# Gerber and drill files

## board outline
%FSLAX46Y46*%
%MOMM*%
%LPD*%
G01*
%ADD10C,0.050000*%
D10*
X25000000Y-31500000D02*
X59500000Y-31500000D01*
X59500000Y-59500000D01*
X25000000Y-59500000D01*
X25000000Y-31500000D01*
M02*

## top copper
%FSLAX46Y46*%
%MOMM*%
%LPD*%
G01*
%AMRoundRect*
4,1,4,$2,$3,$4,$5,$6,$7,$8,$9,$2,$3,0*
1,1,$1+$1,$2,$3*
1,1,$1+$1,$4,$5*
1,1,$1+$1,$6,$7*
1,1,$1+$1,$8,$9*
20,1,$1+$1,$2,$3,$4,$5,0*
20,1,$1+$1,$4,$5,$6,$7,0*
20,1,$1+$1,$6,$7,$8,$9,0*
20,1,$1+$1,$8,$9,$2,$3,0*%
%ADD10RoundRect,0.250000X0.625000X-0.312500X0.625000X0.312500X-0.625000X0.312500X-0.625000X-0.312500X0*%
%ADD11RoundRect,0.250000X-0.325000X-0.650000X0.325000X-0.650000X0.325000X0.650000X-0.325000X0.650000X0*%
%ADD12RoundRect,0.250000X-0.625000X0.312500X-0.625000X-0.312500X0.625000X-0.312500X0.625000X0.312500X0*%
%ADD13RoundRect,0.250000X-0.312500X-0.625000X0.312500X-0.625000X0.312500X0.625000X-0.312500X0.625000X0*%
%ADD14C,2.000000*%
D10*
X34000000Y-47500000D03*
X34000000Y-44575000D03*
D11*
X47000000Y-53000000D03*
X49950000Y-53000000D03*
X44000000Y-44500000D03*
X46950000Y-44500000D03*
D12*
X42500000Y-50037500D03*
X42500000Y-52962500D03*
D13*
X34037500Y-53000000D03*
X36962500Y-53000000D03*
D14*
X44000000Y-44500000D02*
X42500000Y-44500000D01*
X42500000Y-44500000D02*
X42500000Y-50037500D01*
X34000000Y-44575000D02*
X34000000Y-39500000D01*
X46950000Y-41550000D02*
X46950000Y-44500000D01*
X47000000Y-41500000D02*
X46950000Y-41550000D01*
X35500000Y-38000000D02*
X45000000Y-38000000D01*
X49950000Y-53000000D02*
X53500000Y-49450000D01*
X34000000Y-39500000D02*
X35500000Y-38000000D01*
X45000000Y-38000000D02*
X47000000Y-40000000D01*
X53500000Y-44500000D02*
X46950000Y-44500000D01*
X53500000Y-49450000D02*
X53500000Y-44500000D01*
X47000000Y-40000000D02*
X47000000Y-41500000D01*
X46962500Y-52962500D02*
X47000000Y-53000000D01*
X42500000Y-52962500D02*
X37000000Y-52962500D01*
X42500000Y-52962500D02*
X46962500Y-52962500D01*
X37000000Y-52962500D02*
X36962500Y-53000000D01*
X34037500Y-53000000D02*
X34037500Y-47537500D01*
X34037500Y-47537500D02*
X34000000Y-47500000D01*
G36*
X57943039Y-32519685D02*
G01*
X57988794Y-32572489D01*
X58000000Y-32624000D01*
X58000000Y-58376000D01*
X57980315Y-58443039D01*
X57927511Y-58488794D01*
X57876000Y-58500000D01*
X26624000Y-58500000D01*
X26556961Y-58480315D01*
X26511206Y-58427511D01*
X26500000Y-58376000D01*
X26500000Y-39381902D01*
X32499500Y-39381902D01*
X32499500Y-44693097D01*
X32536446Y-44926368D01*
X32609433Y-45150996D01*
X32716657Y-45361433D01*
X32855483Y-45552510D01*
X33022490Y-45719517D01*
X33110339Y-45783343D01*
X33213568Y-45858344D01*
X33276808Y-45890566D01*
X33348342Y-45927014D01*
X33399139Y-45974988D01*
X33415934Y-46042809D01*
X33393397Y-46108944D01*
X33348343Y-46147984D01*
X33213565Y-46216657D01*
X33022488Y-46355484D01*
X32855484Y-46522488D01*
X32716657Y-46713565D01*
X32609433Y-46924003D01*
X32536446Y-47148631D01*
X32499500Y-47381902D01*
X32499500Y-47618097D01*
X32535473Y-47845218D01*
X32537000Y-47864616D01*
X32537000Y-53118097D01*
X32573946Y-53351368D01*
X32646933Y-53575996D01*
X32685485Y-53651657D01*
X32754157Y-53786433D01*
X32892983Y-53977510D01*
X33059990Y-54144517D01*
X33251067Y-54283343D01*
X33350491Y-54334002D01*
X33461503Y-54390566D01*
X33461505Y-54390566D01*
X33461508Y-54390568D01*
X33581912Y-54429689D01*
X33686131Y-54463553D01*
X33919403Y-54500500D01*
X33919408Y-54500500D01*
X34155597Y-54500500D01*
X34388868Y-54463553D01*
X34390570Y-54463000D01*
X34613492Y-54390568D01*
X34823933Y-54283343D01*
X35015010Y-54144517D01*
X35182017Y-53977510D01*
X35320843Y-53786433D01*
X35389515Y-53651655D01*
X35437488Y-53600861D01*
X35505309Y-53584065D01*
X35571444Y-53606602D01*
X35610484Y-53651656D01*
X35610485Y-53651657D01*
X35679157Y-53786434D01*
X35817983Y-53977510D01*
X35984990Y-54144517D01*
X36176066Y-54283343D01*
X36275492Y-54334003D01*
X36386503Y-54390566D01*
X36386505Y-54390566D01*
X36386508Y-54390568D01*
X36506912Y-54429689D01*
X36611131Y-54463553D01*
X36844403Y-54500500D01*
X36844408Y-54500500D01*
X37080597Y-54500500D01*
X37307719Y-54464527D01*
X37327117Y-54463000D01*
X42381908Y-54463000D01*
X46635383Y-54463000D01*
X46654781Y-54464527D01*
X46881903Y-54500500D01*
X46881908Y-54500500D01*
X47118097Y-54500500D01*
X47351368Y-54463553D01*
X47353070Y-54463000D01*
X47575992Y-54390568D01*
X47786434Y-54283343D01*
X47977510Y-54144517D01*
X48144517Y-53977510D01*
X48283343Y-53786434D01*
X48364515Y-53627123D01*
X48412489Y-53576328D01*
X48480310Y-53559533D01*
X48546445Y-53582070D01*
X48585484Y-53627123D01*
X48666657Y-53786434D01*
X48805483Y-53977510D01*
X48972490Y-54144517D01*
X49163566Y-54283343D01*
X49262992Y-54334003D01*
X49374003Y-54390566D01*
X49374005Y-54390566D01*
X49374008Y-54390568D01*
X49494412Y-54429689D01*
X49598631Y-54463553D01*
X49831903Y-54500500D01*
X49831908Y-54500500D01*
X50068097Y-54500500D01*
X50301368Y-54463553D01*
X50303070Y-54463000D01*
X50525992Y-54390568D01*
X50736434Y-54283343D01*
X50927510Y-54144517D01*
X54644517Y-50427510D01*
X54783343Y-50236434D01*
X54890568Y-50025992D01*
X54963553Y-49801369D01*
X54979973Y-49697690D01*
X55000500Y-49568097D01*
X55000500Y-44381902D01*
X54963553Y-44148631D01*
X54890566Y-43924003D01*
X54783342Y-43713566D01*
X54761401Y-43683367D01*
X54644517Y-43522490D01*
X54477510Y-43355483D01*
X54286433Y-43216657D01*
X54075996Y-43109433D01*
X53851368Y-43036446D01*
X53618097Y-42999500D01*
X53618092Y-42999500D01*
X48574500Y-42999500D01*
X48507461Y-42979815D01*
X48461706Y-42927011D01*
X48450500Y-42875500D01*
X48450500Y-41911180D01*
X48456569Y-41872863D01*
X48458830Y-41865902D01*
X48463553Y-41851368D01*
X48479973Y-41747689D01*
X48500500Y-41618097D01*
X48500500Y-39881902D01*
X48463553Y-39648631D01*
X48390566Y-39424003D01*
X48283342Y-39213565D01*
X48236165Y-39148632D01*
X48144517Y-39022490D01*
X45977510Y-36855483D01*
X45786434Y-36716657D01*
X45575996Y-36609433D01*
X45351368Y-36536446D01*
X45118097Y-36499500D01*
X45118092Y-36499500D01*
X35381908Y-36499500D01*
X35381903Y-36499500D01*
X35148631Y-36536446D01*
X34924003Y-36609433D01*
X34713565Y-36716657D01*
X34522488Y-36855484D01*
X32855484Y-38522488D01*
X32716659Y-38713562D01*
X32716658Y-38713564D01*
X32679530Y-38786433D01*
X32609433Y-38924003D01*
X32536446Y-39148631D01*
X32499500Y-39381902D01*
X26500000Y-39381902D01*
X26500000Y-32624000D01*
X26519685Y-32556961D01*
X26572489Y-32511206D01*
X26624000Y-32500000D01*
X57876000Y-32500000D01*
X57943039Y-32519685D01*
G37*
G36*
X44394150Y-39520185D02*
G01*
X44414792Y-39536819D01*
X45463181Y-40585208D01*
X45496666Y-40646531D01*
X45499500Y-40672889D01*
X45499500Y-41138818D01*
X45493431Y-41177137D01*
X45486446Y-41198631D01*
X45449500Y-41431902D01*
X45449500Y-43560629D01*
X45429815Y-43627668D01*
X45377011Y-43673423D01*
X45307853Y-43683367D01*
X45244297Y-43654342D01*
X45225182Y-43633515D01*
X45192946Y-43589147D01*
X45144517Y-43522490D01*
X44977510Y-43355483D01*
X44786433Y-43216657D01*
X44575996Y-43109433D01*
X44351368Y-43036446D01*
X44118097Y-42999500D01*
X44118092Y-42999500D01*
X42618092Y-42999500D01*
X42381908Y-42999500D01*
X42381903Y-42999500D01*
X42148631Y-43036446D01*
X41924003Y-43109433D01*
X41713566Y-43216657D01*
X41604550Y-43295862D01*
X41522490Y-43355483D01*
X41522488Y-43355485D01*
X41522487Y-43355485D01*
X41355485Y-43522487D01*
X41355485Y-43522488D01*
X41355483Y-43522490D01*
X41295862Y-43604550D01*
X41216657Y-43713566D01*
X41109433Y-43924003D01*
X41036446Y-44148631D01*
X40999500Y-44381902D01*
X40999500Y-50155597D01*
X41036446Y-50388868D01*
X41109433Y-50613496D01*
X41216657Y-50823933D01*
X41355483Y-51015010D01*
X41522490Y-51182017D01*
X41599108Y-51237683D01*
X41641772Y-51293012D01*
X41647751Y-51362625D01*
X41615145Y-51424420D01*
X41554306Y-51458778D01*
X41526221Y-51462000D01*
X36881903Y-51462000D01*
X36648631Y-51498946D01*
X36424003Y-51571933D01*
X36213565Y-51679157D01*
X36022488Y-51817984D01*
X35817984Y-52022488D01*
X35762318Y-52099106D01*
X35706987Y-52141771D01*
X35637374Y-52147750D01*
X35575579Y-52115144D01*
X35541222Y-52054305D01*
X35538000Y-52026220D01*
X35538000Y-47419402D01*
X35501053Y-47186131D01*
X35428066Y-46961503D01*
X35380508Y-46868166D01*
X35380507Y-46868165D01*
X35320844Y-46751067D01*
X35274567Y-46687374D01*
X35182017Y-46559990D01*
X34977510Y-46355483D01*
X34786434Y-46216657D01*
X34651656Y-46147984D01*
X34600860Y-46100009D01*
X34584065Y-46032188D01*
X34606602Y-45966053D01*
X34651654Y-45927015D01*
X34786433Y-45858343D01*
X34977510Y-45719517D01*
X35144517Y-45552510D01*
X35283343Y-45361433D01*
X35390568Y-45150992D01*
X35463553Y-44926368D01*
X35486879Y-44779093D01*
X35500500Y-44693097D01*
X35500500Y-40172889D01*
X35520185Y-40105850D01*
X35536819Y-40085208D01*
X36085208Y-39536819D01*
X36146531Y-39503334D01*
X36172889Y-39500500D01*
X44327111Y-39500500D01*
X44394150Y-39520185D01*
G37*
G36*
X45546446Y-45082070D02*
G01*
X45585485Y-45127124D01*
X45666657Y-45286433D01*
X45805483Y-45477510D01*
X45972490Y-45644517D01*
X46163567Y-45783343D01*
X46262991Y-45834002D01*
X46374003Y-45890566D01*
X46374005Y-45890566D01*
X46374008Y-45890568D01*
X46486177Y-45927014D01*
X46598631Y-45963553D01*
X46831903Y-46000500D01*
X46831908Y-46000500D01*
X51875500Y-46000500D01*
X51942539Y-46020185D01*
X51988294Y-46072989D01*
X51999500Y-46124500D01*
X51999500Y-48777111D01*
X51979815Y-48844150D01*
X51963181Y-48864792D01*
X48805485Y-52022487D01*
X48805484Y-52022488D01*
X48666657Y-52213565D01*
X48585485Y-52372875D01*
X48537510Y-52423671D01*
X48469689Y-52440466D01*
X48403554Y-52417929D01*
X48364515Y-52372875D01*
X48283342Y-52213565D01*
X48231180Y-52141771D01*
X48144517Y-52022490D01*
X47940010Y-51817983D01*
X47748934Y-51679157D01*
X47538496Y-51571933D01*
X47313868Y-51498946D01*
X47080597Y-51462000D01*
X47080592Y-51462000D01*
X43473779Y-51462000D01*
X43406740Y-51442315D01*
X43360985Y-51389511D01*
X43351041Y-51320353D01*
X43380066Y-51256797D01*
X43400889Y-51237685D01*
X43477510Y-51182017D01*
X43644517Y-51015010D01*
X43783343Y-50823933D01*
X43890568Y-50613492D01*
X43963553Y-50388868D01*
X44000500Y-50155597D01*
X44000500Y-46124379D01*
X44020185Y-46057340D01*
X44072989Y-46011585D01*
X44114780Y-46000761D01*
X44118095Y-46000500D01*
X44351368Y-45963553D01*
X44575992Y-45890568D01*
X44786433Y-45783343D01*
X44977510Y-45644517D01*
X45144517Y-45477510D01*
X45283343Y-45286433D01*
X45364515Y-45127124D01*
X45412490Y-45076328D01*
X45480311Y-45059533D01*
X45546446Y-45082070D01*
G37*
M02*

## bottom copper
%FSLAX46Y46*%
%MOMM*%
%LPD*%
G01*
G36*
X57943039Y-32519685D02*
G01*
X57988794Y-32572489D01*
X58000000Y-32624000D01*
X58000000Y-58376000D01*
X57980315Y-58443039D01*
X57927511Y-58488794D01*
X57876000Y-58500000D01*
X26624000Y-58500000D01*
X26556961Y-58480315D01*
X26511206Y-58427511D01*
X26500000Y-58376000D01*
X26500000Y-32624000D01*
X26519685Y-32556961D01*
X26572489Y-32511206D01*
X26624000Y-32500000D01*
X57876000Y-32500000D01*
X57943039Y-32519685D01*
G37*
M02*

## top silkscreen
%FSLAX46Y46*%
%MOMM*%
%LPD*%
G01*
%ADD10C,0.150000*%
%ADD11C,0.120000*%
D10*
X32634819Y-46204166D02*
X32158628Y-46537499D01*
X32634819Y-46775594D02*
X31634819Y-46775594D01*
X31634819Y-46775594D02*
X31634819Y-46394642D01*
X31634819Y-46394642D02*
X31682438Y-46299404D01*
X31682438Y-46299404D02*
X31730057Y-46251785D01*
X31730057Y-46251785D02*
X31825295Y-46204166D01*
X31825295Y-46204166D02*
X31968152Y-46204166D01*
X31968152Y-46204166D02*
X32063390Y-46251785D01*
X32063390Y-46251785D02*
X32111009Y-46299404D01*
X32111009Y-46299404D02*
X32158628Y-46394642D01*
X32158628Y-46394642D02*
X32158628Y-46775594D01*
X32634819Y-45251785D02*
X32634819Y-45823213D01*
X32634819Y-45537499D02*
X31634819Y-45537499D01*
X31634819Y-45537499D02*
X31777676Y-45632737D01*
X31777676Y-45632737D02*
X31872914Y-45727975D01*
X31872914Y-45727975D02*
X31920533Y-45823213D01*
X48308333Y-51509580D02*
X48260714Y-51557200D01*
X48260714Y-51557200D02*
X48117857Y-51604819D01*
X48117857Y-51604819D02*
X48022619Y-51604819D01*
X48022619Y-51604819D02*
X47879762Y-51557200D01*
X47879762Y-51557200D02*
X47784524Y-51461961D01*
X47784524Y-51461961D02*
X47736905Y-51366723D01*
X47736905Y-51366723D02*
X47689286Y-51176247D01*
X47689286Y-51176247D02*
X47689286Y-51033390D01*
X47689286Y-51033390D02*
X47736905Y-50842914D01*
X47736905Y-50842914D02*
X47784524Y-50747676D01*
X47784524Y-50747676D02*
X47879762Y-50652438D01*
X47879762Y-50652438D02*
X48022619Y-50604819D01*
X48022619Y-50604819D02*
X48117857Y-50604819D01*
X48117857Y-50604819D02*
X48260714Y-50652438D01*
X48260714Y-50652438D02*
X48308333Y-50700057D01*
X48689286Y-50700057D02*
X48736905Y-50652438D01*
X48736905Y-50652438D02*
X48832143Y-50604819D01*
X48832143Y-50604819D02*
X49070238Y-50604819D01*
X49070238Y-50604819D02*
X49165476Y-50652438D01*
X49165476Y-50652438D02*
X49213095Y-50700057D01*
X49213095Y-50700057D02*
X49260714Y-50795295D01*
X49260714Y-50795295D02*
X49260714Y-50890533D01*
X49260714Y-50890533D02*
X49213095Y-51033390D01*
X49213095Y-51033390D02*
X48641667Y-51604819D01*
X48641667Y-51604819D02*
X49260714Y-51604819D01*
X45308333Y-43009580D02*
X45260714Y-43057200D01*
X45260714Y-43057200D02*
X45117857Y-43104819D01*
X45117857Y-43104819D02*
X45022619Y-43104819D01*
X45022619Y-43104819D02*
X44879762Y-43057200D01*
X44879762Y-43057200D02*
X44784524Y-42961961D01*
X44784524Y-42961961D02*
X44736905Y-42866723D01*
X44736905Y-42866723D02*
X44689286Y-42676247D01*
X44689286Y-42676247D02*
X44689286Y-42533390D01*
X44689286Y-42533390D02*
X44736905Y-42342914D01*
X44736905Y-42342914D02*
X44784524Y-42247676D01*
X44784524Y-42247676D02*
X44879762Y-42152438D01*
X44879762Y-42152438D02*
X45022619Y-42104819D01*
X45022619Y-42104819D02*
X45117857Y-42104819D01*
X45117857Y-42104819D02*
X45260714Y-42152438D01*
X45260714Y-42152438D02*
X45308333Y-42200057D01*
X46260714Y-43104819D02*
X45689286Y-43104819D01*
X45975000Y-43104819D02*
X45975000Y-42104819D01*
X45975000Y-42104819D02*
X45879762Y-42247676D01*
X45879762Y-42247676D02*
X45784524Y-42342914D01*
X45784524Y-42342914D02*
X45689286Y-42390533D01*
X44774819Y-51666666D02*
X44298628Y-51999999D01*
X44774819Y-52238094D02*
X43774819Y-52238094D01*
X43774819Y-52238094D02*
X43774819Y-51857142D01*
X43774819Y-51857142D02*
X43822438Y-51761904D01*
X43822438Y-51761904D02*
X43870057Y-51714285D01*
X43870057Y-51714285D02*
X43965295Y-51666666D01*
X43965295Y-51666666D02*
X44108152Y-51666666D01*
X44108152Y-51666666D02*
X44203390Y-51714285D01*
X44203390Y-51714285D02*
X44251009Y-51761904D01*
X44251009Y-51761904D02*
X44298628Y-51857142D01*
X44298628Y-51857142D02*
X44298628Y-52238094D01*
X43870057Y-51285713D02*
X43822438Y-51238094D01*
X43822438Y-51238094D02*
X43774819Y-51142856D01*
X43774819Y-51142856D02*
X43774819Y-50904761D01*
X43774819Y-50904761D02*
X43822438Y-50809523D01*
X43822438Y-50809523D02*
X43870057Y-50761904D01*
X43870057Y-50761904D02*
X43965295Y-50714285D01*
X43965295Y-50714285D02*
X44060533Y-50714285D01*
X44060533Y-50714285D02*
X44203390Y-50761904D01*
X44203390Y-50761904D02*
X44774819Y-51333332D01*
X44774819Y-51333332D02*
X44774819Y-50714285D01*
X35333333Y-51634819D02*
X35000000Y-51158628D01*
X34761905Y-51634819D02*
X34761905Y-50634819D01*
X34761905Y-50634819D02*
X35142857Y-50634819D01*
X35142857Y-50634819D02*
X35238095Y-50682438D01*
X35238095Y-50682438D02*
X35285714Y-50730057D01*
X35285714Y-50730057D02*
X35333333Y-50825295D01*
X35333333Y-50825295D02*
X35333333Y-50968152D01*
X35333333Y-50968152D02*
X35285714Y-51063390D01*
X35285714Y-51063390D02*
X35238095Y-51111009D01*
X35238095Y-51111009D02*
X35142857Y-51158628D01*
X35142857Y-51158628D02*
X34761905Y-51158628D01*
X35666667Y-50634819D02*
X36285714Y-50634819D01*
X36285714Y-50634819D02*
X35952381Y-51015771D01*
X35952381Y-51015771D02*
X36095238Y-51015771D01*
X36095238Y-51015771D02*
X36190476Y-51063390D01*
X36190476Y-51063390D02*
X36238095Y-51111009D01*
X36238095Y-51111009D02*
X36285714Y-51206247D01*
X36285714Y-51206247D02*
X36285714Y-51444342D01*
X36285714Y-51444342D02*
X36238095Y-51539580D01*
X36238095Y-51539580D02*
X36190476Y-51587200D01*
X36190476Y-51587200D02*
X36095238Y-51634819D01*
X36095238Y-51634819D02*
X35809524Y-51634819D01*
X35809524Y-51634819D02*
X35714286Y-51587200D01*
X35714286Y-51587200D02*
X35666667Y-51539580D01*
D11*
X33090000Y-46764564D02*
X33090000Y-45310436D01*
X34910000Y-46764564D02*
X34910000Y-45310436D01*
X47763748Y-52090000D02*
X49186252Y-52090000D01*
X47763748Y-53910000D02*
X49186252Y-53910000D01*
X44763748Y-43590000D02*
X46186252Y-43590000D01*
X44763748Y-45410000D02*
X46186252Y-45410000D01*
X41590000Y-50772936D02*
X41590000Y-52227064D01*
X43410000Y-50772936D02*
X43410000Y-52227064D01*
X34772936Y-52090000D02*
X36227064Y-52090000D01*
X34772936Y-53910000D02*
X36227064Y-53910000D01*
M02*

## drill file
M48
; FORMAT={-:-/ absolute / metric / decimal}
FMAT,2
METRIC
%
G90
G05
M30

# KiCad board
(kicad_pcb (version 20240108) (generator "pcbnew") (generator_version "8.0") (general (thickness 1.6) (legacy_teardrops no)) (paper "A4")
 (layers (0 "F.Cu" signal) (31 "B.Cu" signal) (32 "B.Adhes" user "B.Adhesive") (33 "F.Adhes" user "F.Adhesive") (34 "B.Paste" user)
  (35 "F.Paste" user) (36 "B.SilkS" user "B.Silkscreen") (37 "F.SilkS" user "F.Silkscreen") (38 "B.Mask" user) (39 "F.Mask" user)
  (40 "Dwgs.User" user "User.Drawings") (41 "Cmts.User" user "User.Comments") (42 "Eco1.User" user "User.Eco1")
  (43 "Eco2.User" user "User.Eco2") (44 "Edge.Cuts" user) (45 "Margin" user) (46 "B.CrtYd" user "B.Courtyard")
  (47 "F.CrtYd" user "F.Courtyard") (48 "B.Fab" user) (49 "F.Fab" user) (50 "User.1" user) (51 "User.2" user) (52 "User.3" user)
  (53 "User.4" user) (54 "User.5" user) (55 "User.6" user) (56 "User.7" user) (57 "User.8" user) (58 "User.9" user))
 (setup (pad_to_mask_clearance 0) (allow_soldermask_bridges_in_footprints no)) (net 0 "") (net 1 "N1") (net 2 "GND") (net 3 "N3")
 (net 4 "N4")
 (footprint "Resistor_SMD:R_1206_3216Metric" (layer "F.Cu") (at 34 46.0375 90)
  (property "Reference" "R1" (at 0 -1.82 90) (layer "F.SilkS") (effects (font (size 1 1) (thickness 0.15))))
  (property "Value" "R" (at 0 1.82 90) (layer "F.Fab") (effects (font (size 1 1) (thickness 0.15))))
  (fp_line (start -0.727064 -0.91) (end 0.727064 -0.91) (stroke (width 0.12) (type solid)) (layer "F.SilkS"))
  (fp_line (start -0.727064 0.91) (end 0.727064 0.91) (stroke (width 0.12) (type solid)) (layer "F.SilkS"))
  (pad "1" smd roundrect (at -1.4625 0 90) (size 1.125 1.75) (layers "F.Cu" "F.Paste" "F.Mask") (roundrect_rratio 0.222222) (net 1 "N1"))
  (pad "2" smd roundrect (at 1.4625 0 90) (size 1.125 1.75) (layers "F.Cu" "F.Paste" "F.Mask") (roundrect_rratio 0.222222) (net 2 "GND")))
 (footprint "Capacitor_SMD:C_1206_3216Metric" (layer "F.Cu") (at 48.475 53)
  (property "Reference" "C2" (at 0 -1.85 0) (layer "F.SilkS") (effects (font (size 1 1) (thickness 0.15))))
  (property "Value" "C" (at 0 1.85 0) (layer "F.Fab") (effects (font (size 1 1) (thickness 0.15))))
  (fp_line (start -0.711252 -0.91) (end 0.711252 -0.91) (stroke (width 0.12) (type solid)) (layer "F.SilkS"))
  (fp_line (start -0.711252 0.91) (end 0.711252 0.91) (stroke (width 0.12) (type solid)) (layer "F.SilkS"))
  (pad "1" smd roundrect (at -1.475 0) (size 1.15 1.8) (layers "F.Cu" "F.Paste" "F.Mask") (roundrect_rratio 0.217391) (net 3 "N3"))
  (pad "2" smd roundrect (at 1.475 0) (size 1.15 1.8) (layers "F.Cu" "F.Paste" "F.Mask") (roundrect_rratio 0.217391) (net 2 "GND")))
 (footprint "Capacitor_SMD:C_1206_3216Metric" (layer "F.Cu") (at 45.475 44.5)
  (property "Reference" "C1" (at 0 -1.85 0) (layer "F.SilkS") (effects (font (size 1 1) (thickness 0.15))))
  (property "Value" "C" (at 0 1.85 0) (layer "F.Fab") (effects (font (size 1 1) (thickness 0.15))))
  (fp_line (start -0.711252 -0.91) (end 0.711252 -0.91) (stroke (width 0.12) (type solid)) (layer "F.SilkS"))
  (fp_line (start -0.711252 0.91) (end 0.711252 0.91) (stroke (width 0.12) (type solid)) (layer "F.SilkS"))
  (pad "1" smd roundrect (at -1.475 0) (size 1.15 1.8) (layers "F.Cu" "F.Paste" "F.Mask") (roundrect_rratio 0.217391) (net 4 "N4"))
  (pad "2" smd roundrect (at 1.475 0) (size 1.15 1.8) (layers "F.Cu" "F.Paste" "F.Mask") (roundrect_rratio 0.217391) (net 2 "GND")))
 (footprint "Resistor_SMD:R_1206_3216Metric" (layer "F.Cu") (at 42.5 51.5 -90)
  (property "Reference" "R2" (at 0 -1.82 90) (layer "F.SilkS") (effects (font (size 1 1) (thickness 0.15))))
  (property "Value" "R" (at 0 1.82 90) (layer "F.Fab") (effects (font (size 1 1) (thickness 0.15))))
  (fp_line (start -0.727064 0.91) (end 0.727064 0.91) (stroke (width 0.12) (type solid)) (layer "F.SilkS"))
  (fp_line (start -0.727064 -0.91) (end 0.727064 -0.91) (stroke (width 0.12) (type solid)) (layer "F.SilkS"))
  (pad "1" smd roundrect (at -1.4625 0 270) (size 1.125 1.75) (layers "F.Cu" "F.Paste" "F.Mask") (roundrect_rratio 0.222222) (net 4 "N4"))
  (pad "2" smd roundrect (at 1.4625 0 270) (size 1.125 1.75) (layers "F.Cu" "F.Paste" "F.Mask") (roundrect_rratio 0.222222) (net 3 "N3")))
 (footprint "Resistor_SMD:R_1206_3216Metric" (layer "F.Cu") (at 35.5 53)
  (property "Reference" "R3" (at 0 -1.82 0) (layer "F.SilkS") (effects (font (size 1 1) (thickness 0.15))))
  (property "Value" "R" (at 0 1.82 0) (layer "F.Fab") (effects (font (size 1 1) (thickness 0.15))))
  (fp_line (start -0.727064 -0.91) (end 0.727064 -0.91) (stroke (width 0.12) (type solid)) (layer "F.SilkS"))
  (fp_line (start -0.727064 0.91) (end 0.727064 0.91) (stroke (width 0.12) (type solid)) (layer "F.SilkS"))
  (pad "1" smd roundrect (at -1.4625 0) (size 1.125 1.75) (layers "F.Cu" "F.Paste" "F.Mask") (roundrect_rratio 0.222222) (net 1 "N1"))
  (pad "2" smd roundrect (at 1.4625 0) (size 1.125 1.75) (layers "F.Cu" "F.Paste" "F.Mask") (roundrect_rratio 0.222222) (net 3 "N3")))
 (gr_rect (start 25 31.5) (end 59.5 59.5) (stroke (width 0.05) (type default)) (fill none) (layer "Edge.Cuts"))
 (segment (start 44 44.5) (end 42.5 44.5) (width 2) (layer "F.Cu") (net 4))
 (segment (start 42.5 44.5) (end 42.5 50.0375) (width 2) (layer "F.Cu") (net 4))
 (segment (start 34 44.575) (end 34 39.5) (width 2) (layer "F.Cu") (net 2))
 (segment (start 46.95 41.55) (end 46.95 44.5) (width 2) (layer "F.Cu") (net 2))
 (segment (start 47 41.5) (end 46.95 41.55) (width 2) (layer "F.Cu") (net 2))
 (segment (start 35.5 38) (end 45 38) (width 2) (layer "F.Cu") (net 2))
 (segment (start 49.95 53) (end 53.5 49.45) (width 2) (layer "F.Cu") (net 2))
 (segment (start 34 39.5) (end 35.5 38) (width 2) (layer "F.Cu") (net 2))
 (segment (start 45 38) (end 47 40) (width 2) (layer "F.Cu") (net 2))
 (segment (start 53.5 44.5) (end 46.95 44.5) (width 2) (layer "F.Cu") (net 2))
 (segment (start 53.5 49.45) (end 53.5 44.5) (width 2) (layer "F.Cu") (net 2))
 (segment (start 47 40) (end 47 41.5) (width 2) (layer "F.Cu") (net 2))
 (segment (start 46.9625 52.9625) (end 47 53) (width 2) (layer "F.Cu") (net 3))
 (segment (start 42.5 52.9625) (end 37 52.9625) (width 2) (layer "F.Cu") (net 3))
 (segment (start 42.5 52.9625) (end 46.9625 52.9625) (width 2) (layer "F.Cu") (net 3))
 (segment (start 37 52.9625) (end 36.9625 53) (width 2) (layer "F.Cu") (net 3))
 (segment (start 34.0375 53) (end 34.0375 47.5375) (width 2) (layer "F.Cu") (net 1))
 (segment (start 34.0375 47.5375) (end 34 47.5) (width 2) (layer "F.Cu") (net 1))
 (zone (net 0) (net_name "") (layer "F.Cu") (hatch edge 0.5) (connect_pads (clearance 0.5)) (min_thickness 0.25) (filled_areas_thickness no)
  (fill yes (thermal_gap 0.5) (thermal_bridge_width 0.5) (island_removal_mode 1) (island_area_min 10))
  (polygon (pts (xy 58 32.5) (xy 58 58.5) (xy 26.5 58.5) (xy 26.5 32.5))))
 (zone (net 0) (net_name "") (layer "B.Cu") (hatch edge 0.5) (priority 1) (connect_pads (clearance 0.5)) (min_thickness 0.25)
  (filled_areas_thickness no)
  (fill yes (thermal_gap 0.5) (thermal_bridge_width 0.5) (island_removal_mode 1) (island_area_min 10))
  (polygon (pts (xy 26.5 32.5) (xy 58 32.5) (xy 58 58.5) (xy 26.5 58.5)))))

